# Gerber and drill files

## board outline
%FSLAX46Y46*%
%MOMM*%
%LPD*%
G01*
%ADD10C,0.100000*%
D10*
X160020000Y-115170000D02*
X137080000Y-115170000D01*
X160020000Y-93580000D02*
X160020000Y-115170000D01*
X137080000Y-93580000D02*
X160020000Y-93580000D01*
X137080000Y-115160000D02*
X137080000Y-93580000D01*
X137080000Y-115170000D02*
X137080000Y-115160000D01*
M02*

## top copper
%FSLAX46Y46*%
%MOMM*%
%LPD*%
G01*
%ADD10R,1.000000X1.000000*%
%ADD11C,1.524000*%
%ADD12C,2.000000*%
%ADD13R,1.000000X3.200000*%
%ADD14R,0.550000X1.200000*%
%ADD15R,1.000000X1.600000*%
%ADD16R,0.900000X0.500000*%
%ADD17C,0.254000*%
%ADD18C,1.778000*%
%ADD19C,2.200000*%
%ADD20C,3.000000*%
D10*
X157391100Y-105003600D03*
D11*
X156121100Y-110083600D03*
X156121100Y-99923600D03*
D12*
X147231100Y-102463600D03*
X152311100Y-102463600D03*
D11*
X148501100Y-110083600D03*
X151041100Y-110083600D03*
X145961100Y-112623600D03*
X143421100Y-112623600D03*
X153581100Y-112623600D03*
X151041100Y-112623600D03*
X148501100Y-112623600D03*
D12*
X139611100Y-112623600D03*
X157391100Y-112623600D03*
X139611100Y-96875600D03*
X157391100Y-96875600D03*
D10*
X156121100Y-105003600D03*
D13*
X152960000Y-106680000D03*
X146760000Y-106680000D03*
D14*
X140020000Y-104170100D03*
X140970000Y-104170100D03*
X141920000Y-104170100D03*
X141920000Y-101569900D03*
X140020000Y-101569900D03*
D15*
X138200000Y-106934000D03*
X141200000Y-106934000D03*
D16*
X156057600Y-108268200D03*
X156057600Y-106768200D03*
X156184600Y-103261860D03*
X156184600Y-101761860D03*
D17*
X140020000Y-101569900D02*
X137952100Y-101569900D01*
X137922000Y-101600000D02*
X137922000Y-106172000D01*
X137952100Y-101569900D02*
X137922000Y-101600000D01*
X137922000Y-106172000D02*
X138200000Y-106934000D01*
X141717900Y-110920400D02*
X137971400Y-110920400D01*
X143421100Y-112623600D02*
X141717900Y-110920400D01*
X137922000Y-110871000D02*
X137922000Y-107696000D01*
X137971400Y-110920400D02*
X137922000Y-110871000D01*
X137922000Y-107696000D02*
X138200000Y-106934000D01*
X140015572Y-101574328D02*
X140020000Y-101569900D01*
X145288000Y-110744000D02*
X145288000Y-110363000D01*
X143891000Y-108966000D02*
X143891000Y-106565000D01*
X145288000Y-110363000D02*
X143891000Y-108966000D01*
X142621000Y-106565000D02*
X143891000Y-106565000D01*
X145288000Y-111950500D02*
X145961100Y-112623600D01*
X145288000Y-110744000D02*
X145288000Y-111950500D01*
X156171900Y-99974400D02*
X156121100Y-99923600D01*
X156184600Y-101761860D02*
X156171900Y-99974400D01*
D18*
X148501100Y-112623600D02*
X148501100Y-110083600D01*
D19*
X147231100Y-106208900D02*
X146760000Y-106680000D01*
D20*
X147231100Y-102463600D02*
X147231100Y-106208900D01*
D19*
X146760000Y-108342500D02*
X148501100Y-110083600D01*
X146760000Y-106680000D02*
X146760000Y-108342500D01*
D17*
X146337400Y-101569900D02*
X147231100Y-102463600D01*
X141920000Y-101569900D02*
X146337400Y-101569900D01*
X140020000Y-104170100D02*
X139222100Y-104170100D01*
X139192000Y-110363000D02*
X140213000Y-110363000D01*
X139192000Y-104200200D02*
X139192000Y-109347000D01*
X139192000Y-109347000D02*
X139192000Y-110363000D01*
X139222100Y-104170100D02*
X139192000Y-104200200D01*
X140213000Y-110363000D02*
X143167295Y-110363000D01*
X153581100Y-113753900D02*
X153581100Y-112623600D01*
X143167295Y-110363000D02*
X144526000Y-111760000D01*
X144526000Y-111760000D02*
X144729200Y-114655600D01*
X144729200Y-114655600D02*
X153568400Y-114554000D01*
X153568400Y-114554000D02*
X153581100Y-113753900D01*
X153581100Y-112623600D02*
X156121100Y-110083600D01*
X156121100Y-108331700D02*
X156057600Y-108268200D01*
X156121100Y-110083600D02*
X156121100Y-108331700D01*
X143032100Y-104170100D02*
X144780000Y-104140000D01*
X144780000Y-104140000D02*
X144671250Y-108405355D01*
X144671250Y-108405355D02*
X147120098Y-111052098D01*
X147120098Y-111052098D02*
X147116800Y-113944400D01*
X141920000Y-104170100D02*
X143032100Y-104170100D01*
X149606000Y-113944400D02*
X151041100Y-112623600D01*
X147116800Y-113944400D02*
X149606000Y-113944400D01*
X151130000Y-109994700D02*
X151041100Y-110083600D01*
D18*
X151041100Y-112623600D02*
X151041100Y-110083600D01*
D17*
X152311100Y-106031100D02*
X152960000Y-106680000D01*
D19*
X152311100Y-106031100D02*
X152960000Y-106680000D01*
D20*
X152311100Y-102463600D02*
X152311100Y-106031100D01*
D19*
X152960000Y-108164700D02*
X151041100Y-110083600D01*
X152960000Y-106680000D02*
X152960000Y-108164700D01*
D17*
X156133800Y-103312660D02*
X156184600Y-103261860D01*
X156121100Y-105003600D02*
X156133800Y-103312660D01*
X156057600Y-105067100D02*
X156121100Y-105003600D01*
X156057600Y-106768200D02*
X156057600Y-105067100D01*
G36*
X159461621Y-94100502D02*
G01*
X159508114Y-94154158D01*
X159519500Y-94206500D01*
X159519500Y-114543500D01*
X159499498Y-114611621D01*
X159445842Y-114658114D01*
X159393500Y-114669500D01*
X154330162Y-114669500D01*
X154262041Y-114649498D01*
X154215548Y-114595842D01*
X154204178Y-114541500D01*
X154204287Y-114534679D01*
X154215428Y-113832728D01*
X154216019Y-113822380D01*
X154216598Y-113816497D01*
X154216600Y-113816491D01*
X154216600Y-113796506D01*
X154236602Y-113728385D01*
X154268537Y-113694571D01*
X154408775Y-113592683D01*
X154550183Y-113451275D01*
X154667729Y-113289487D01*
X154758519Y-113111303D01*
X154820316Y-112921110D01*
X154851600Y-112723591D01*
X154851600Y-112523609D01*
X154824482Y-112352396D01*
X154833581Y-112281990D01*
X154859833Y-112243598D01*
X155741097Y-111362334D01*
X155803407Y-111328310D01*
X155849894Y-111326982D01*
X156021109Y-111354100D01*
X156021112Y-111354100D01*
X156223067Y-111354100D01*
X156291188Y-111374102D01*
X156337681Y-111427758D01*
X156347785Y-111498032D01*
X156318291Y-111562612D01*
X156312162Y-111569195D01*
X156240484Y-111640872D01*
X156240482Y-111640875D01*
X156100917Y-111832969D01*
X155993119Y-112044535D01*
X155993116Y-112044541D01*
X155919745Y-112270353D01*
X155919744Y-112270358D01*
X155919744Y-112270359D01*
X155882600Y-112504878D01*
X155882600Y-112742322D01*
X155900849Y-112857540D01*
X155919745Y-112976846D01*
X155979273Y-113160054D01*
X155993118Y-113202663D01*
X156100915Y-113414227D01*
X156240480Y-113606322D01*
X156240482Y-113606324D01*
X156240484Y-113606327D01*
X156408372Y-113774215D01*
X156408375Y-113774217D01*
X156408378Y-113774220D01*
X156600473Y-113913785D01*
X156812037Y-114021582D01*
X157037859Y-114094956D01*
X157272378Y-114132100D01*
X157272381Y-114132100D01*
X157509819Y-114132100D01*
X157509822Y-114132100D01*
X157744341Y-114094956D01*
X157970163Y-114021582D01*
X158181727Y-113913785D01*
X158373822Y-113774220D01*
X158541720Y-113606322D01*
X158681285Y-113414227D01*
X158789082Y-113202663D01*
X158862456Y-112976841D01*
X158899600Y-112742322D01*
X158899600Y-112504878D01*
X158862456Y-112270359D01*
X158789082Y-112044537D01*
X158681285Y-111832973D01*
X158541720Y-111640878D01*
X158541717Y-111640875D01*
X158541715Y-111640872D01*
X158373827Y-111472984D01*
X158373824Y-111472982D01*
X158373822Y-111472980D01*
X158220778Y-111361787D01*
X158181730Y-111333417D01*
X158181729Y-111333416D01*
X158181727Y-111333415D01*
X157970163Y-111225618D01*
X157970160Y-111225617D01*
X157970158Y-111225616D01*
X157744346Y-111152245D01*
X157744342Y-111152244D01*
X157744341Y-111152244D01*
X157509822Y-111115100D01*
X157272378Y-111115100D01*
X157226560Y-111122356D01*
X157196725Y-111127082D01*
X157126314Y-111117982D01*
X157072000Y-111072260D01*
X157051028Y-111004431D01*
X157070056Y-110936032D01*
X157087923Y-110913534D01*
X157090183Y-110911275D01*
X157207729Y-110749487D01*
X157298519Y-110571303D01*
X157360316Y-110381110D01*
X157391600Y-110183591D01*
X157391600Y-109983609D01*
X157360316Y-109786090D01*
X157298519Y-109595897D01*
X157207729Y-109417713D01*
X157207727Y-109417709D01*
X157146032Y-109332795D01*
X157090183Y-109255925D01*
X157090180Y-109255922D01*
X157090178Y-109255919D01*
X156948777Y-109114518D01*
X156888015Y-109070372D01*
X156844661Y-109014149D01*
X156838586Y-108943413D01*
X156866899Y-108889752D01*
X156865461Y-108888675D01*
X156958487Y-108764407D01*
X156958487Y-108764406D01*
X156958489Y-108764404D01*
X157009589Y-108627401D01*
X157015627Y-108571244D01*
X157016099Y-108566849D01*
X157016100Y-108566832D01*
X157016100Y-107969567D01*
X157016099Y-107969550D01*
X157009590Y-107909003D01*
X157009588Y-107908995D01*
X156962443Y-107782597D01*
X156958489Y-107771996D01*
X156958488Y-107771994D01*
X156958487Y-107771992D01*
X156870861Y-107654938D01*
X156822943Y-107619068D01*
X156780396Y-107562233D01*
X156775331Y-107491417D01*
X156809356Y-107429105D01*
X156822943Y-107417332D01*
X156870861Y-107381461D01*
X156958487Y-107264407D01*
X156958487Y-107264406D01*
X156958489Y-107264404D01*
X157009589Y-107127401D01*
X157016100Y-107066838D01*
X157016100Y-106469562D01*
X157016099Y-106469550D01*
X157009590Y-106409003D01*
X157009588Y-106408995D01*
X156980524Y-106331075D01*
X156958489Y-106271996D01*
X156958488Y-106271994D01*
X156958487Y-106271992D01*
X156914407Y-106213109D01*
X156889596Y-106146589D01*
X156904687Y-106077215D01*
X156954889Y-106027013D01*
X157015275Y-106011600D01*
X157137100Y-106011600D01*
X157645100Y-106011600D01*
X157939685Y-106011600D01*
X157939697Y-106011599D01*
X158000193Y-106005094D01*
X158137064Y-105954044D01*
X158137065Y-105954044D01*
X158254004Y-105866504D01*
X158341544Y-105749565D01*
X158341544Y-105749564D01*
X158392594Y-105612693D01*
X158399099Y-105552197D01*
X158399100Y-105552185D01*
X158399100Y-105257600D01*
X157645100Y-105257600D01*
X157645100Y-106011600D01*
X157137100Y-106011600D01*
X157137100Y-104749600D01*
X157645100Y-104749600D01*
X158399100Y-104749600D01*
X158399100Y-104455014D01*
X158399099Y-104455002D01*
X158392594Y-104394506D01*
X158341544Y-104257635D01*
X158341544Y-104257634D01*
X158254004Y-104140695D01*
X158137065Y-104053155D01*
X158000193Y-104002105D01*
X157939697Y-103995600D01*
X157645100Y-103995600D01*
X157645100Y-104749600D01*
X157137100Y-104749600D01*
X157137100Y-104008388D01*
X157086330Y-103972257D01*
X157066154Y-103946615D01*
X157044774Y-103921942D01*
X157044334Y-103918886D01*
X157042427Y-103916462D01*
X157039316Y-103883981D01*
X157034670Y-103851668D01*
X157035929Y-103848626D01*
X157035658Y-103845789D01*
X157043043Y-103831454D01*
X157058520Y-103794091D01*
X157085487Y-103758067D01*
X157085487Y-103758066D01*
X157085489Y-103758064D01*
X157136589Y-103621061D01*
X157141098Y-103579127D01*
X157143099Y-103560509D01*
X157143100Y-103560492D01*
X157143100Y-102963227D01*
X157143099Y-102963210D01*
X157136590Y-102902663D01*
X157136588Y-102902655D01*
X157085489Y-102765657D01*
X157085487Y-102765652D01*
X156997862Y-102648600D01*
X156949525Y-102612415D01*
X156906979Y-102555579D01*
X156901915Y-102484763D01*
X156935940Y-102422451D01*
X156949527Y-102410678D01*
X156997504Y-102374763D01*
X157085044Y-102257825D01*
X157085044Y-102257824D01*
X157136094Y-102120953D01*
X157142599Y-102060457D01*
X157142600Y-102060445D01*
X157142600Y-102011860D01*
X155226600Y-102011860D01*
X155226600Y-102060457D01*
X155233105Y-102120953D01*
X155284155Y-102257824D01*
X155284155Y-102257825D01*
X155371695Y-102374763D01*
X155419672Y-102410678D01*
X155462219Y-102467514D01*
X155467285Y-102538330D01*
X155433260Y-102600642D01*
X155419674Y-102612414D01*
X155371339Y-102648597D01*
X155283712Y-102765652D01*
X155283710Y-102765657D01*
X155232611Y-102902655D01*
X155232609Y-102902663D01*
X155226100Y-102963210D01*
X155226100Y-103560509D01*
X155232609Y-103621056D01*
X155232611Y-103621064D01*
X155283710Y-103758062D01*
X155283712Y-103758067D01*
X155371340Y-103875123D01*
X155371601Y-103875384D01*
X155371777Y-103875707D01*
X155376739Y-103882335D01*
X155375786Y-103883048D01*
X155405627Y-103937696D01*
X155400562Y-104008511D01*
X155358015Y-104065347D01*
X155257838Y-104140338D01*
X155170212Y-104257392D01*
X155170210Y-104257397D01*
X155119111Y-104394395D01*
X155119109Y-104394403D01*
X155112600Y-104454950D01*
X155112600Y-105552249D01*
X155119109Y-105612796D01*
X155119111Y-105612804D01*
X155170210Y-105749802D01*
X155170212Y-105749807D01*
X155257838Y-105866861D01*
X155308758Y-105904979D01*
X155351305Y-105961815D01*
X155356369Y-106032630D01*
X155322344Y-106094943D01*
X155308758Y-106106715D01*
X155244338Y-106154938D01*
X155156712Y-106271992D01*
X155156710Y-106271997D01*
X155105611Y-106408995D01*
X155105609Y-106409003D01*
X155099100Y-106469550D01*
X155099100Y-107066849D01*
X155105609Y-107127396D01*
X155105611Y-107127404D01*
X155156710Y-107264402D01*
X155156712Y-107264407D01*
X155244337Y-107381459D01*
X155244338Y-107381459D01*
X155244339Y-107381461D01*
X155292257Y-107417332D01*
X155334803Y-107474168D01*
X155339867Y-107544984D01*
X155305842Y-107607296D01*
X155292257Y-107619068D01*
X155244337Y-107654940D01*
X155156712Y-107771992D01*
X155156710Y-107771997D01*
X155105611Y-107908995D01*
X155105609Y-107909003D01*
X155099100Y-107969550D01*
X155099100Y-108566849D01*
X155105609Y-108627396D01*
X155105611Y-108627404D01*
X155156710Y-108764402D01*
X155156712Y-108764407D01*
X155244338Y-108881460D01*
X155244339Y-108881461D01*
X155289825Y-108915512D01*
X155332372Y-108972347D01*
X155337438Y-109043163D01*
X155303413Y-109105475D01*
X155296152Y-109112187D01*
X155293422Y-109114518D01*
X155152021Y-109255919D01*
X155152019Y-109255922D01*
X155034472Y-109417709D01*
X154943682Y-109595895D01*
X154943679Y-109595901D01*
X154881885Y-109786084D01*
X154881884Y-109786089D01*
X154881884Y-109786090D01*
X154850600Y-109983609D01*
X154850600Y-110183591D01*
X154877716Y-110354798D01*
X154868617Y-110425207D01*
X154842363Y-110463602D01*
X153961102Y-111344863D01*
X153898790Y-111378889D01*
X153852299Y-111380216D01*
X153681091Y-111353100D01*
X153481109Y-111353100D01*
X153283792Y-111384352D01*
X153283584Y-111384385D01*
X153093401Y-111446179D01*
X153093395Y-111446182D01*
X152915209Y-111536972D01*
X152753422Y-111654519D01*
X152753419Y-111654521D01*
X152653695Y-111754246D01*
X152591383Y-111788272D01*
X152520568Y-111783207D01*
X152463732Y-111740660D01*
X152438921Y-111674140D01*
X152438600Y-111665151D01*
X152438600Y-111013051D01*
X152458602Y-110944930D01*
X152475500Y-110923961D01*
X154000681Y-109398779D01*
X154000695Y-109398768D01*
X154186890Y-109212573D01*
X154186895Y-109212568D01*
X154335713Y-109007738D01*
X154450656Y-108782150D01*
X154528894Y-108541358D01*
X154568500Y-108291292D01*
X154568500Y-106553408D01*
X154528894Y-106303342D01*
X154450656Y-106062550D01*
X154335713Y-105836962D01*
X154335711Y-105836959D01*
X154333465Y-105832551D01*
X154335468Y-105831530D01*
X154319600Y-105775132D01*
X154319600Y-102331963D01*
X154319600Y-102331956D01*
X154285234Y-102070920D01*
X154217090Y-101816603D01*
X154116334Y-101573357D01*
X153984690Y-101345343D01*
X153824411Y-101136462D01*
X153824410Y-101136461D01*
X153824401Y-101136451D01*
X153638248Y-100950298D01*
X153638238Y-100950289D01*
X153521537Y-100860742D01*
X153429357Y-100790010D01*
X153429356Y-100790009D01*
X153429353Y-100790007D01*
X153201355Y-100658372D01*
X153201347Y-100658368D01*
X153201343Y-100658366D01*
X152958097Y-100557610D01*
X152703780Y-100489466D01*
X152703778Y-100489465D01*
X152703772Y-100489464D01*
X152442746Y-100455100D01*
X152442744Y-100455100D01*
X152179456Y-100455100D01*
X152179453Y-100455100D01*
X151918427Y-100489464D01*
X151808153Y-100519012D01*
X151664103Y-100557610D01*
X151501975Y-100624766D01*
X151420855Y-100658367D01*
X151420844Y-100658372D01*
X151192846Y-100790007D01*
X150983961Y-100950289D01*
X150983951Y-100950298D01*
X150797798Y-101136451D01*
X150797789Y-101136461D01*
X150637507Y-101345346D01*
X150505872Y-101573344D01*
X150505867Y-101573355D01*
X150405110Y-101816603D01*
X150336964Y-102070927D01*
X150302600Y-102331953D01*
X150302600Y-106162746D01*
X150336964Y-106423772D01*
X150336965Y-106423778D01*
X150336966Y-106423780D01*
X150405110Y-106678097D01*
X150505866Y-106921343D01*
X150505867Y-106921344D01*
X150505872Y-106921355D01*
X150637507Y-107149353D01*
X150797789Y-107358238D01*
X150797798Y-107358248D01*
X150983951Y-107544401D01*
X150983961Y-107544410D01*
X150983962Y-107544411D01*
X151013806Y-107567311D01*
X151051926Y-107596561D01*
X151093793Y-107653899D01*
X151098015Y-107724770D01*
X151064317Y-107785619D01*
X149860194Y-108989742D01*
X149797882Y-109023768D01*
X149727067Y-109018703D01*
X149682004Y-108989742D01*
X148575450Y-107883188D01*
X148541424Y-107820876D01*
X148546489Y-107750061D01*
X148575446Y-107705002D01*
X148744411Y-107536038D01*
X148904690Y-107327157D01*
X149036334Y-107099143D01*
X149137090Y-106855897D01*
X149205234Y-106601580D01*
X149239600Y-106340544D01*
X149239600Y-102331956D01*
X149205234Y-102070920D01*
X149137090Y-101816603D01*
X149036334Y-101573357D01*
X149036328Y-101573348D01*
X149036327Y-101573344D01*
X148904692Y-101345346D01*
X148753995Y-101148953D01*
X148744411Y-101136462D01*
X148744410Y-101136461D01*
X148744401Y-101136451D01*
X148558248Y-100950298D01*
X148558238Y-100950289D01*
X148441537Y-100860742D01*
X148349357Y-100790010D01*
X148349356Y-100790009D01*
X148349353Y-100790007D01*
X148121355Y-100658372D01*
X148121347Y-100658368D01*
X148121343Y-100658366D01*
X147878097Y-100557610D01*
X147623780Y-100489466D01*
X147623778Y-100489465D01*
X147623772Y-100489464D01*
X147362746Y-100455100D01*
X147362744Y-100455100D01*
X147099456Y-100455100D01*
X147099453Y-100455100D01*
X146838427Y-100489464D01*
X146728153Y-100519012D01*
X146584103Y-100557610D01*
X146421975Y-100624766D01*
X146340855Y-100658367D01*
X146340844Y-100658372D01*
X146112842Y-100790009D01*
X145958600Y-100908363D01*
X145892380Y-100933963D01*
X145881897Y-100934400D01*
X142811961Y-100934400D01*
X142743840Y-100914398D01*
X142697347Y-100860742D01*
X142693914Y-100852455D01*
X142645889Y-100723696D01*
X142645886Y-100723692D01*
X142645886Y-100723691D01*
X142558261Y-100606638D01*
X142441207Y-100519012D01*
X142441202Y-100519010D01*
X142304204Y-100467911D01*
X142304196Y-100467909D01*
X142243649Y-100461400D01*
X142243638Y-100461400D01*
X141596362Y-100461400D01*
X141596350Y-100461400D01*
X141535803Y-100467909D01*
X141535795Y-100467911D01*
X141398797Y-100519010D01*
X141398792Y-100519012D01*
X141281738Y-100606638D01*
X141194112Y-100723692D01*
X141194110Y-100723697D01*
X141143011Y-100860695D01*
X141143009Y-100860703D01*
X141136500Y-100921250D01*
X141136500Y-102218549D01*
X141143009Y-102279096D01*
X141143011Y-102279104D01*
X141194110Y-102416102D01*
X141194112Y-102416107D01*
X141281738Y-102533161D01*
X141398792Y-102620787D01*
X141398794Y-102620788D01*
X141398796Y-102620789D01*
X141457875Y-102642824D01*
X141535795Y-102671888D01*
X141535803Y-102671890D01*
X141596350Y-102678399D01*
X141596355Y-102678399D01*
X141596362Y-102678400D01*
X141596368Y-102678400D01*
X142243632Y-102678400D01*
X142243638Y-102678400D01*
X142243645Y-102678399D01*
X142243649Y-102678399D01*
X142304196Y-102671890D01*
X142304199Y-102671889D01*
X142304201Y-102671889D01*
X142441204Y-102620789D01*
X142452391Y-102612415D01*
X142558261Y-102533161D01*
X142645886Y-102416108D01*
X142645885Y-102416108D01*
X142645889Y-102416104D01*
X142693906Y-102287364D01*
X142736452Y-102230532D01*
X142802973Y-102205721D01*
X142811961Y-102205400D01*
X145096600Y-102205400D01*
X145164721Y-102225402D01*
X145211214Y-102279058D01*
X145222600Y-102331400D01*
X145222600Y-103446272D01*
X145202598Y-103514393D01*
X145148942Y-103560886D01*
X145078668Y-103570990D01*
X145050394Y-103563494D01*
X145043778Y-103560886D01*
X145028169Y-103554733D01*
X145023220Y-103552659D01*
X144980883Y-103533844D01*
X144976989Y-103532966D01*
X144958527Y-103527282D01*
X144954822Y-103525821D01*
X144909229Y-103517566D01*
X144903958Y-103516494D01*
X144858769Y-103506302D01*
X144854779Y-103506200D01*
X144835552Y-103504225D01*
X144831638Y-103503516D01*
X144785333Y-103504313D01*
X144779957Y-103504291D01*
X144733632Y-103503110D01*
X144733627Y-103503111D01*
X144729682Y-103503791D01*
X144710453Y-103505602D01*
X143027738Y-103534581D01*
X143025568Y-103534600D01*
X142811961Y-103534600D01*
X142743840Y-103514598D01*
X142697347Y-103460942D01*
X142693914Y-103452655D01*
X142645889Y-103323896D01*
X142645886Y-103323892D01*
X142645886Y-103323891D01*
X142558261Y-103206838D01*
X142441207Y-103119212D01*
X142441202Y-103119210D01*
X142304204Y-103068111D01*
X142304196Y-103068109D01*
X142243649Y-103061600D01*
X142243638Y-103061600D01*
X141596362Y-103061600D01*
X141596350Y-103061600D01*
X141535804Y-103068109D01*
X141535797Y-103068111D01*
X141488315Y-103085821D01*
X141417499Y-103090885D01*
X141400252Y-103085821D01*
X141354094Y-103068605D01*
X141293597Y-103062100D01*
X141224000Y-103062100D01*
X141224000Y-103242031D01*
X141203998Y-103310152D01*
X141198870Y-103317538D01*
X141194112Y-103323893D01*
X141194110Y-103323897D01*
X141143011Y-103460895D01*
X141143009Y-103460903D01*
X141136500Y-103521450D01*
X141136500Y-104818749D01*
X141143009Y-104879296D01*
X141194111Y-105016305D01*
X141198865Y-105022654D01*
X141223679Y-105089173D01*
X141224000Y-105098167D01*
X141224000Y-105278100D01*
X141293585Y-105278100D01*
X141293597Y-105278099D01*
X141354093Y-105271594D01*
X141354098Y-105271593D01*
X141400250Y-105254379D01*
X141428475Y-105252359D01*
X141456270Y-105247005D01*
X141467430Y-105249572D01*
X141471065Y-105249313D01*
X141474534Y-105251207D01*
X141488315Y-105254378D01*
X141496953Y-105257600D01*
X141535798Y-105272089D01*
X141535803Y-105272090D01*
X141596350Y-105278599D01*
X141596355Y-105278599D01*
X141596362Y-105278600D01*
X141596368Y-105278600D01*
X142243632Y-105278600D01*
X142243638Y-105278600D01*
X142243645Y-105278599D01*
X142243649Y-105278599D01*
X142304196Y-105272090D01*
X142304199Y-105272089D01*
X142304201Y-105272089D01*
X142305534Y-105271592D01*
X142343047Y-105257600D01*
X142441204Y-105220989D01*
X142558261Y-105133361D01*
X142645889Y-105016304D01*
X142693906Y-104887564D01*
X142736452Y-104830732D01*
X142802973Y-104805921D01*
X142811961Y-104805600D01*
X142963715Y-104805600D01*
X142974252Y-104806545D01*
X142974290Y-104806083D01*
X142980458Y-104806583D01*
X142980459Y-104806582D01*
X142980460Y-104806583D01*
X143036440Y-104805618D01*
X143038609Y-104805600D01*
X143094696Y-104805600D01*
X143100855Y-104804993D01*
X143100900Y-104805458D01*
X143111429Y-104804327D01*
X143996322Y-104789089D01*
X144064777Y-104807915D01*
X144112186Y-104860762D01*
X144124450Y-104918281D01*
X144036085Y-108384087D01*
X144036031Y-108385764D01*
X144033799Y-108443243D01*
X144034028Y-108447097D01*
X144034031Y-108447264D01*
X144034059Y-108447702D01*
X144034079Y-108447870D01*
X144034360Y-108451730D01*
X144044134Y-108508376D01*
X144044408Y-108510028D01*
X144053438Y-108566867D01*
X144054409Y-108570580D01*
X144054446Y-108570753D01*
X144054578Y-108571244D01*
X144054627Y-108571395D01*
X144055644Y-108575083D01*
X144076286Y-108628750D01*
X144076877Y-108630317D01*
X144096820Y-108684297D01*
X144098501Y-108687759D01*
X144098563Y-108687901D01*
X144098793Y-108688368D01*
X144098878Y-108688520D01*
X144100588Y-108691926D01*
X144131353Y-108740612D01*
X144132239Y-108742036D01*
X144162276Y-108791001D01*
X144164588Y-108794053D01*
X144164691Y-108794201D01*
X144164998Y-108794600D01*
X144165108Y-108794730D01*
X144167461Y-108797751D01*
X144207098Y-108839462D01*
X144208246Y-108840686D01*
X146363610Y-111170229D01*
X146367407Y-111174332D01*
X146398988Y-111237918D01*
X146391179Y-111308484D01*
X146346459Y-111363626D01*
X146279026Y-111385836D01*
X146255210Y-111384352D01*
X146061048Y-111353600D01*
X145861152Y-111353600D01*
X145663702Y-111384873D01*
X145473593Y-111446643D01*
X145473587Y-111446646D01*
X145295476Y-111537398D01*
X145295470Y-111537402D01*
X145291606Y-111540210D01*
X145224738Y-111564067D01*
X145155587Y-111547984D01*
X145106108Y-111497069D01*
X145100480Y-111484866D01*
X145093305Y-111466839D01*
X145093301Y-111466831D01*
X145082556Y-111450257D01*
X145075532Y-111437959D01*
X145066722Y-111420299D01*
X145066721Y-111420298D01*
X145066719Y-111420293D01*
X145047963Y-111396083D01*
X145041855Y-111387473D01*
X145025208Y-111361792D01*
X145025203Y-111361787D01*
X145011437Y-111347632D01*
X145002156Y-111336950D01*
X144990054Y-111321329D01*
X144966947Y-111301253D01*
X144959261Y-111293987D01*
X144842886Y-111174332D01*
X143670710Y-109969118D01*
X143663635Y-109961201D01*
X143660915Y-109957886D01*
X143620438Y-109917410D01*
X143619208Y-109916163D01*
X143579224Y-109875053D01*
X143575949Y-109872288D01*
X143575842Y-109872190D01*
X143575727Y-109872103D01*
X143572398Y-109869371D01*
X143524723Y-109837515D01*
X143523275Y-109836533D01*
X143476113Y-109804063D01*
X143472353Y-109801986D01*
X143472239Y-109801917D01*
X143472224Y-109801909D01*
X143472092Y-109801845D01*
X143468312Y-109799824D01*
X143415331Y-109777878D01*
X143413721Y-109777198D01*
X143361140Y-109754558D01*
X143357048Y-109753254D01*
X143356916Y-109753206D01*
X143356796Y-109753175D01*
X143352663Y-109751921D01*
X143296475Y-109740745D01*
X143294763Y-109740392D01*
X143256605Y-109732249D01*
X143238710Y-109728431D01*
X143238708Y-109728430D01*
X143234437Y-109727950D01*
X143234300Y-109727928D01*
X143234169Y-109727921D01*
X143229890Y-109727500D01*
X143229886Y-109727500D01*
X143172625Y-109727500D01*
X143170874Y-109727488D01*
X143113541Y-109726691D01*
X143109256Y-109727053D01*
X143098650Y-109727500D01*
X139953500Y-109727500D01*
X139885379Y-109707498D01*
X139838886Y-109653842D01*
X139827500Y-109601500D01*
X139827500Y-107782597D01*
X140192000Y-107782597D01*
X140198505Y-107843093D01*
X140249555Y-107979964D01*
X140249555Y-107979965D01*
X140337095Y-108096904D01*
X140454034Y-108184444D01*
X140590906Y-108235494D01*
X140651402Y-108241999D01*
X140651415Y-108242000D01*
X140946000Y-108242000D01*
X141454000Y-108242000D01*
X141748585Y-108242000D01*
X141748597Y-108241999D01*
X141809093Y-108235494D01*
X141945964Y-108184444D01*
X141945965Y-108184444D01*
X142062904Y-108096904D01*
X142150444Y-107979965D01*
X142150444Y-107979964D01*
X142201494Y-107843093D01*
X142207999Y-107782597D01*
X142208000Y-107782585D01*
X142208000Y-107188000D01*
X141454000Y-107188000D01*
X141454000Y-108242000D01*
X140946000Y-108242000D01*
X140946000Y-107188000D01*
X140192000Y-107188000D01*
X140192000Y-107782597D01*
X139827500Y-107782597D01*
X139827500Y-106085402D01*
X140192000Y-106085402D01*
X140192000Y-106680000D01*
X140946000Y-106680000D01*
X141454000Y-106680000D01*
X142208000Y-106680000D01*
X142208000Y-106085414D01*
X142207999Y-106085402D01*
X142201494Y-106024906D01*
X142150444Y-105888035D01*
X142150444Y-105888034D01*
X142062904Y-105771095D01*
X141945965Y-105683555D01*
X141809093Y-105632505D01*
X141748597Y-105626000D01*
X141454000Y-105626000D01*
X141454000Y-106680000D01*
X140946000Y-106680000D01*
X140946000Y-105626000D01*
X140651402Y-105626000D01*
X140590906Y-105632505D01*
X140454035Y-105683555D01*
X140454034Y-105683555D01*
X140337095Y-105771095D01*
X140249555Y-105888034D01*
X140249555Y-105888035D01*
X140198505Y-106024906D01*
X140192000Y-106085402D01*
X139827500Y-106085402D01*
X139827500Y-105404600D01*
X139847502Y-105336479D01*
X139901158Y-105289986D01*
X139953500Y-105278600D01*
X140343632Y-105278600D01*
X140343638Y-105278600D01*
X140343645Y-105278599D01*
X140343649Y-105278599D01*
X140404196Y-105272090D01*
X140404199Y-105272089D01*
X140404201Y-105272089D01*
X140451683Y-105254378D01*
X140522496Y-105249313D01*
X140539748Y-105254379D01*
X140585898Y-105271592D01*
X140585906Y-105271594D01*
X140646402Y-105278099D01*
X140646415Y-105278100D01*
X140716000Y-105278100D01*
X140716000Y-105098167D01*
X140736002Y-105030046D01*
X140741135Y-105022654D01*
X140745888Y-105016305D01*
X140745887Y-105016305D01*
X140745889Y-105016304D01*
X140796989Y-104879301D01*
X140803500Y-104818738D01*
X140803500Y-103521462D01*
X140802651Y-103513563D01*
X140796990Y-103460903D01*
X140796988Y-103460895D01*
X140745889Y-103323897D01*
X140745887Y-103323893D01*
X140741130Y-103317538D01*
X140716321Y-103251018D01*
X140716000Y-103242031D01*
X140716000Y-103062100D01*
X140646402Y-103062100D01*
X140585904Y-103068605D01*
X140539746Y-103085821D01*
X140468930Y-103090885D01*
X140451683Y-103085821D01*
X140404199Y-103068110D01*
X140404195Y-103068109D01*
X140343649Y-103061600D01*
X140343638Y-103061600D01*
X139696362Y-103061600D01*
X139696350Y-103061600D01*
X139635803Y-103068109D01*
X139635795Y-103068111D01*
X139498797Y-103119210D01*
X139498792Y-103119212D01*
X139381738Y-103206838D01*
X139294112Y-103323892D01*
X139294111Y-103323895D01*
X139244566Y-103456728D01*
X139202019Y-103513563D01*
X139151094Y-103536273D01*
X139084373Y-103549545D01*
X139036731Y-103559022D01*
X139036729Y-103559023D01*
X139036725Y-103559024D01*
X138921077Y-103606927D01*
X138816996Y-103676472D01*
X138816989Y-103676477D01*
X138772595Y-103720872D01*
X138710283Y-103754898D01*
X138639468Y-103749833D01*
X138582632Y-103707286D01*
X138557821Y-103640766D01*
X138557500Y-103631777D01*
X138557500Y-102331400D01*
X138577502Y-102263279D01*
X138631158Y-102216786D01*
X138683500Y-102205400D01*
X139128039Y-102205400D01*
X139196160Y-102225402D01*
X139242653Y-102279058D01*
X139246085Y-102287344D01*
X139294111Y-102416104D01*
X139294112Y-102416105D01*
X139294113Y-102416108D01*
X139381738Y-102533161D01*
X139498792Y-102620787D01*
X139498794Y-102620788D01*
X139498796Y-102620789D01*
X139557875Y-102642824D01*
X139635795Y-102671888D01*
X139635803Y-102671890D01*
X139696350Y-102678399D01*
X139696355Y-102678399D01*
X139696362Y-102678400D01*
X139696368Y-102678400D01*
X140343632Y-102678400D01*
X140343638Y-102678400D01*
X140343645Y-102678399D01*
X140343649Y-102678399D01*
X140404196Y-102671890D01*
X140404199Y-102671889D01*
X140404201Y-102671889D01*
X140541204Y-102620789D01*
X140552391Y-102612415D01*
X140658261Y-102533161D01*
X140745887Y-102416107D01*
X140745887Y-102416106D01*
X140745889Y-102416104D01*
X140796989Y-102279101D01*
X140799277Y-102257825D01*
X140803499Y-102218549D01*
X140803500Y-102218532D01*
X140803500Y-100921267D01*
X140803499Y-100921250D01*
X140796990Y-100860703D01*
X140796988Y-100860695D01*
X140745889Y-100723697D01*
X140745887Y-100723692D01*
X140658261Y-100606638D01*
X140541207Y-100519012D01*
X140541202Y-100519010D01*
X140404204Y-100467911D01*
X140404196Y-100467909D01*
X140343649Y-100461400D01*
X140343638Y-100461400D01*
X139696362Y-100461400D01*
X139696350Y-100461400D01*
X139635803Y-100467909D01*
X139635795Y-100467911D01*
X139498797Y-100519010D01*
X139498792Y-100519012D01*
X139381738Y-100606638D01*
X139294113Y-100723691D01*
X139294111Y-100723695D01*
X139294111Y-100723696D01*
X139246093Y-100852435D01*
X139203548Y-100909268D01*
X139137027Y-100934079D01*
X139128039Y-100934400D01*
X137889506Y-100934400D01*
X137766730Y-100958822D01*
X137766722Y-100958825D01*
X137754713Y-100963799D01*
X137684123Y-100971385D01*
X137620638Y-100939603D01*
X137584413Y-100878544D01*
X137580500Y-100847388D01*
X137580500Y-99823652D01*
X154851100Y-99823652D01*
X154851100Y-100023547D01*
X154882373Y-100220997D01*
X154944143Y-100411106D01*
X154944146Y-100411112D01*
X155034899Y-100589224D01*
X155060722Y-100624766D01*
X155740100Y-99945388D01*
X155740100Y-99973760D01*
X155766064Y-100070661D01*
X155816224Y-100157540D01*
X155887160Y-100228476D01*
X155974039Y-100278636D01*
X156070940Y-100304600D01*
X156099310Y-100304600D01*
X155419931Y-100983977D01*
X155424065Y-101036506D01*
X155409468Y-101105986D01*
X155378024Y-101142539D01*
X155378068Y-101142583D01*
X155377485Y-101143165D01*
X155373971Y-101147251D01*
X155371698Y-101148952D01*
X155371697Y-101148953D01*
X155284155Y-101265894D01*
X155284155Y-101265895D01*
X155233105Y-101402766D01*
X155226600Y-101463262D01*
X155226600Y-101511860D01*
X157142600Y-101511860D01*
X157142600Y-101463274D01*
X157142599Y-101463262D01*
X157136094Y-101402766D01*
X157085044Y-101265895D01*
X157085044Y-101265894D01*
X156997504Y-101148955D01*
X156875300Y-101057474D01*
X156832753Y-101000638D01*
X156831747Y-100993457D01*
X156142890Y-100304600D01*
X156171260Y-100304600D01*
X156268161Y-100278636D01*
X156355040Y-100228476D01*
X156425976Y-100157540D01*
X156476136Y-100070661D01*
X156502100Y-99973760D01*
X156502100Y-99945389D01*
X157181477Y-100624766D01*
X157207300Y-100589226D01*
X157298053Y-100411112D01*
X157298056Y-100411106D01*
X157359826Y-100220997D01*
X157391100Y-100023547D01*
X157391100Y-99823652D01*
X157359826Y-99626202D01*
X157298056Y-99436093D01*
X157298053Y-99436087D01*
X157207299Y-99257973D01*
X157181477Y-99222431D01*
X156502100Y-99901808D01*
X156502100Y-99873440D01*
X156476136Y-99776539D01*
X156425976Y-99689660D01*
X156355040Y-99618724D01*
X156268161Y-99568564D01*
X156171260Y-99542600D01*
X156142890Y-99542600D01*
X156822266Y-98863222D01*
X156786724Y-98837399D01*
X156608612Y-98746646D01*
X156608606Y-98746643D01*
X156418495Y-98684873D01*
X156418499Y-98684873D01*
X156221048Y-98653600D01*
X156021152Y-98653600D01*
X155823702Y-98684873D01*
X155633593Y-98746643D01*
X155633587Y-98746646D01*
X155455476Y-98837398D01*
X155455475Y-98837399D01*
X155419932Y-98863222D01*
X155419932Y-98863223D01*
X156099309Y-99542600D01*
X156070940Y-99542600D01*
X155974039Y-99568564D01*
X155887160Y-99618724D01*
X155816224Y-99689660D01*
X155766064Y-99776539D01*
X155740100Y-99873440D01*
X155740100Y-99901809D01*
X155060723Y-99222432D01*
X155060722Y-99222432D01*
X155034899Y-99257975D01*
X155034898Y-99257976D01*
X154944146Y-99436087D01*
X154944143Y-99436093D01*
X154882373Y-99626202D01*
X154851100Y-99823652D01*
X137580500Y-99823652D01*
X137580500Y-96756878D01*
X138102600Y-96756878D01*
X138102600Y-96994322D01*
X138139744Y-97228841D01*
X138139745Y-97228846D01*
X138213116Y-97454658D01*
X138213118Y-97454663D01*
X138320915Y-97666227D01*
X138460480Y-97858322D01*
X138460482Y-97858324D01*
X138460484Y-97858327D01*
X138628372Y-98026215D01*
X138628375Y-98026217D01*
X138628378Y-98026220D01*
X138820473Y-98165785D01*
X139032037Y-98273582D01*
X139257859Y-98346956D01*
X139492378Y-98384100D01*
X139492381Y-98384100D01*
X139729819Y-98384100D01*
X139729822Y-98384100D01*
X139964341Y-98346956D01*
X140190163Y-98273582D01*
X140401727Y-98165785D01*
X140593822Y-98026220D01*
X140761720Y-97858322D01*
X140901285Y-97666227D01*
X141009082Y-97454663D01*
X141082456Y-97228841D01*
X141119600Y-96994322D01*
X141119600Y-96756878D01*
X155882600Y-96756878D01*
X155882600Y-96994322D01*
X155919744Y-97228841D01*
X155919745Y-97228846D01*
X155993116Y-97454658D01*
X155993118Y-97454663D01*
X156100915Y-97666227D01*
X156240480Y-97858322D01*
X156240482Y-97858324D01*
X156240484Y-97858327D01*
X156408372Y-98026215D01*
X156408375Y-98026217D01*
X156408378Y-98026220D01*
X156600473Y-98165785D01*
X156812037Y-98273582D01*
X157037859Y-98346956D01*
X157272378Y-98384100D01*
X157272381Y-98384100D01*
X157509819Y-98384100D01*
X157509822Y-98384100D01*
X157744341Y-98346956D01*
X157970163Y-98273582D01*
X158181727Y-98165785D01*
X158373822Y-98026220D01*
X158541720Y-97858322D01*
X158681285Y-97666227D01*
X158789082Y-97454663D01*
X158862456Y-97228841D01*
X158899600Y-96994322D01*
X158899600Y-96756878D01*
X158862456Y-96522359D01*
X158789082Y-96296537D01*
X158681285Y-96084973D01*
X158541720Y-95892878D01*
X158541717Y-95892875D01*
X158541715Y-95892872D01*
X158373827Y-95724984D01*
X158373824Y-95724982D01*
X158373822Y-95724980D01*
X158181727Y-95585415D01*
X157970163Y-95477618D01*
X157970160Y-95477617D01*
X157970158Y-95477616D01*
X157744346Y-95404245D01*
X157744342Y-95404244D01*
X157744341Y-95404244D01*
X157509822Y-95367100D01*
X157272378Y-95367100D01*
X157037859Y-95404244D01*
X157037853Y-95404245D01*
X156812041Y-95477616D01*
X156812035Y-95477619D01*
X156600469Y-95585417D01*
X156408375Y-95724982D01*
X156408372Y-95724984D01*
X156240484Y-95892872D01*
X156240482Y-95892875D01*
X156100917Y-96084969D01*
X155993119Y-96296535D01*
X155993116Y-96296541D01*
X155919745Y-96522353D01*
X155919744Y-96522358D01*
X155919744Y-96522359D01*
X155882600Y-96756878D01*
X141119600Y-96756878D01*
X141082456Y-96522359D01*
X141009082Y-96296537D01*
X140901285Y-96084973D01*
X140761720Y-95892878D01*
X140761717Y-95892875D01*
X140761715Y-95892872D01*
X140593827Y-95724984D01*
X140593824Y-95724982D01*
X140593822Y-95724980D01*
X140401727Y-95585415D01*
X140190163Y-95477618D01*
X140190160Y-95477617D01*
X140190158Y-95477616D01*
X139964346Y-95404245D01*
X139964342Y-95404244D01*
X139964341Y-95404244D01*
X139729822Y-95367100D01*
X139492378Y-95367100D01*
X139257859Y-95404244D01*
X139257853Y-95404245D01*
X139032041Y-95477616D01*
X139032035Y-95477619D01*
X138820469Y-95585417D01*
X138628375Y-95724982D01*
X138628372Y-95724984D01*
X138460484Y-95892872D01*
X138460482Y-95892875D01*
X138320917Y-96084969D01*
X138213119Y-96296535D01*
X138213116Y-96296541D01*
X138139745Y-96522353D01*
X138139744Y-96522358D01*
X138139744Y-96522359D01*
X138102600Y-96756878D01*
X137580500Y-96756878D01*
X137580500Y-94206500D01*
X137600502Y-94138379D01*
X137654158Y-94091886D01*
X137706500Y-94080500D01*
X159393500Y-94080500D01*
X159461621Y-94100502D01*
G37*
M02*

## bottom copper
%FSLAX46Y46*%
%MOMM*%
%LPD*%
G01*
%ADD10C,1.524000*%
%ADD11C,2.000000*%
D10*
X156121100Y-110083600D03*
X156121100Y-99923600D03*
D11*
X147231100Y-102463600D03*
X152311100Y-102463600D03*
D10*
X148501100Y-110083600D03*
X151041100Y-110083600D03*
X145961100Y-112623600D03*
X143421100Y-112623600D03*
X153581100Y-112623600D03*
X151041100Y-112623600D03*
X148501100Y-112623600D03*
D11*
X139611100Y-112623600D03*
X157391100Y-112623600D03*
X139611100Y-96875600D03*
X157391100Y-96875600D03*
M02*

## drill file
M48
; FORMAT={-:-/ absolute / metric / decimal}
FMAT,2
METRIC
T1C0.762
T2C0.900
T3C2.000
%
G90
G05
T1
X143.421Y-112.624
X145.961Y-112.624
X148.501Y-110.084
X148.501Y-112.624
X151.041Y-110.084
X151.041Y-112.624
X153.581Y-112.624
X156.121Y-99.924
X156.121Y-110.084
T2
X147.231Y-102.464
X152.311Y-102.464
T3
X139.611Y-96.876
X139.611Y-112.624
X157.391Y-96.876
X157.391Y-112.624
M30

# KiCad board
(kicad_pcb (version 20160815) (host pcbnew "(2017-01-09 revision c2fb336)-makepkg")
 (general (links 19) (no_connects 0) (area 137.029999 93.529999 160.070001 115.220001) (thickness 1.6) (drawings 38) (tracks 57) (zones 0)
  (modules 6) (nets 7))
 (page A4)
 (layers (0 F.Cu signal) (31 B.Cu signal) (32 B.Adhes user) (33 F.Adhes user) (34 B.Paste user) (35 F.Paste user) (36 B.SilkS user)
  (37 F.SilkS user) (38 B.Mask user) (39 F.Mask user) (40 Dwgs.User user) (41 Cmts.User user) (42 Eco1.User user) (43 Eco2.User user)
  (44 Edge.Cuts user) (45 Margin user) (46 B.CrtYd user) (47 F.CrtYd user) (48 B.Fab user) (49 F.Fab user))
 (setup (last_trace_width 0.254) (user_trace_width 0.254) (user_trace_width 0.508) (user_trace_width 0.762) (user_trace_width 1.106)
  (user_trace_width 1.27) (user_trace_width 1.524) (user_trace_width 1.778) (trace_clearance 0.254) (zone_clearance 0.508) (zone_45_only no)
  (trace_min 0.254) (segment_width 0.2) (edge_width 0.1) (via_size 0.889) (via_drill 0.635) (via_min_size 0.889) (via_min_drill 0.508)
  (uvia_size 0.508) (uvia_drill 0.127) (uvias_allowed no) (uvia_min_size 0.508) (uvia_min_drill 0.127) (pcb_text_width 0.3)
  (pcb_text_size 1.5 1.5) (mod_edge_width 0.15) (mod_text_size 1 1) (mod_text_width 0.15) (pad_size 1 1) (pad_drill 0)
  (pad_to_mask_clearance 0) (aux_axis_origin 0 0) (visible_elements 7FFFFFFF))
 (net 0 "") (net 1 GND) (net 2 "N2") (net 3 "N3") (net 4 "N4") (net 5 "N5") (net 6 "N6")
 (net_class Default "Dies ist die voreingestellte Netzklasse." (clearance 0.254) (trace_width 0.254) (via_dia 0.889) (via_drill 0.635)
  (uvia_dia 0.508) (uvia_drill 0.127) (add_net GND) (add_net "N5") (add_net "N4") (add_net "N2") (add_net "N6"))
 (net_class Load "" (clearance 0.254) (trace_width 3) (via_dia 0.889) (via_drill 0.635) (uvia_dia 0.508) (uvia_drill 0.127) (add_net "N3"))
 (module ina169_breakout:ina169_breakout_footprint (layer F.Cu) (at 148.5011 105.0036)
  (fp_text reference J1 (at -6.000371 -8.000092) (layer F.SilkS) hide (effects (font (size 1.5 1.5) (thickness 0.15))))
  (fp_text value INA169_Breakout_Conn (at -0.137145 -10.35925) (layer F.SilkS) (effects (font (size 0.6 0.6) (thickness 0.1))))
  (pad 2 smd rect (at 8.89 0) (size 1 1) (layers F.Cu F.Paste F.Mask) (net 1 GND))
  (pad 5 thru_hole circle (at 7.62 5.08) (size 1.524 1.524) (drill 0.762) (layers *.Cu *.Mask F.SilkS) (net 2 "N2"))
  (pad 2 thru_hole circle (at 7.62 -5.08) (size 1.524 1.524) (drill 0.762) (layers *.Cu *.Mask F.SilkS) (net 1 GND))
  (pad 3 thru_hole circle (at -1.27 -2.54) (size 2 2) (drill 0.9) (layers *.Cu *.Mask F.SilkS) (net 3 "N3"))
  (pad 4 thru_hole circle (at 3.81 -2.54) (size 2 2) (drill 0.9) (layers *.Cu *.Mask F.SilkS) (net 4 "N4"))
  (pad 3 thru_hole circle (at 0 5.08) (size 1.524 1.524) (drill 0.762) (layers *.Cu *.Mask F.SilkS) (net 3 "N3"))
  (pad 4 thru_hole circle (at 2.54 5.08) (size 1.524 1.524) (drill 0.762) (layers *.Cu *.Mask F.SilkS) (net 4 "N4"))
  (pad 2 thru_hole circle (at -2.54 7.62) (size 1.524 1.524) (drill 0.762) (layers *.Cu *.Mask F.SilkS) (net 1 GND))
  (pad 1 thru_hole circle (at -5.08 7.62) (size 1.524 1.524) (drill 0.762) (layers *.Cu *.Mask F.SilkS) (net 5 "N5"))
  (pad 5 thru_hole circle (at 5.08 7.62) (size 1.524 1.524) (drill 0.762) (layers *.Cu *.Mask F.SilkS) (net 2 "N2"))
  (pad 4 thru_hole circle (at 2.54 7.62) (size 1.524 1.524) (drill 0.762) (layers *.Cu *.Mask F.SilkS) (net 4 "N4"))
  (pad 3 thru_hole circle (at 0 7.62) (size 1.524 1.524) (drill 0.762) (layers *.Cu *.Mask F.SilkS) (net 3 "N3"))
  (pad "" thru_hole circle (at -8.89 7.62) (size 2 2) (drill 2) (layers *.Cu *.Mask F.SilkS))
  (pad "" thru_hole circle (at 8.89 7.62) (size 2 2) (drill 2) (layers *.Cu *.Mask F.SilkS))
  (pad "" thru_hole circle (at -8.89 -8.128) (size 2 2) (drill 2) (layers *.Cu *.Mask F.SilkS))
  (pad "" thru_hole circle (at 8.89 -8.128) (size 2 2) (drill 2) (layers *.Cu *.Mask F.SilkS))
  (pad 6 smd rect (at 7.62 0) (size 1 1) (layers F.Cu F.Paste F.Mask)))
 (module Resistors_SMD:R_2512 (layer F.Cu) (at 149.86 106.68 180)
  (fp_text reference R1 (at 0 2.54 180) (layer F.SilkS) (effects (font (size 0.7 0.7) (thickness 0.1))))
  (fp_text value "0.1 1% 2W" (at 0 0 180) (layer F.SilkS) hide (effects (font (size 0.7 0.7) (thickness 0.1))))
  (pad 1 smd rect (at -3.1 0 180) (size 1 3.2) (layers F.Cu F.Paste F.Mask) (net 4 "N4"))
  (pad 2 smd rect (at 3.1 0 180) (size 1 3.2) (layers F.Cu F.Paste F.Mask) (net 3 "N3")))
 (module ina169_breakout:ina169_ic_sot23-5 (layer F.Cu) (at 140.97 102.87)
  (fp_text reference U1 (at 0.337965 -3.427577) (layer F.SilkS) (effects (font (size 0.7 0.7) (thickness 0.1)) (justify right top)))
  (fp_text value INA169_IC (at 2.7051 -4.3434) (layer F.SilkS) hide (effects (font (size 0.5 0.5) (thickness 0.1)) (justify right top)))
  (pad 1 smd rect (at -0.95 1.3001) (size 0.55 1.2) (layers F.Cu F.Paste F.Mask) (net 2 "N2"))
  (pad 2 smd rect (at 0 1.3001) (size 0.55 1.2) (layers F.Cu F.Paste F.Mask) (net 1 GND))
  (pad 3 smd rect (at 0.95 1.3001) (size 0.55 1.2) (layers F.Cu F.Paste F.Mask) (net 4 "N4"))
  (pad 4 smd rect (at 0.95 -1.3001) (size 0.55 1.2) (layers F.Cu F.Paste F.Mask) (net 3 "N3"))
  (pad 5 smd rect (at -0.95 -1.3001) (size 0.55 1.2) (layers F.Cu F.Paste F.Mask) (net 5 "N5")))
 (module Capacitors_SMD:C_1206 (layer F.Cu) (at 139.7 106.934)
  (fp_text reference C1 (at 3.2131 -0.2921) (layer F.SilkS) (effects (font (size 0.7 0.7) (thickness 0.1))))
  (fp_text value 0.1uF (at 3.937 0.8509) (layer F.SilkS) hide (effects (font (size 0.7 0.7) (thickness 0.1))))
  (pad 1 smd rect (at -1.5 0) (size 1 1.6) (layers F.Cu F.Paste F.Mask) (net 5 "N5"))
  (pad 2 smd rect (at 1.5 0) (size 1 1.6) (layers F.Cu F.Paste F.Mask) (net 1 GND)))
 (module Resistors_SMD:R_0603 (layer F.Cu) (at 156.0576 107.5182 90)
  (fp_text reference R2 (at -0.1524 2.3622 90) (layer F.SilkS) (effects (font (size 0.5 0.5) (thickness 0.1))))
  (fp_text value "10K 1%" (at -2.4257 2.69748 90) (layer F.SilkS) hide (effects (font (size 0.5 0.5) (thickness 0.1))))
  (pad 1 smd rect (at -0.75 0 90) (size 0.5 0.9) (layers F.Cu F.Paste F.Mask) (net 2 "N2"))
  (pad 2 smd rect (at 0.75 0 90) (size 0.5 0.9) (layers F.Cu F.Paste F.Mask) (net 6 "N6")))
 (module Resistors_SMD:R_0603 (layer F.Cu) (at 156.1846 102.51186 90)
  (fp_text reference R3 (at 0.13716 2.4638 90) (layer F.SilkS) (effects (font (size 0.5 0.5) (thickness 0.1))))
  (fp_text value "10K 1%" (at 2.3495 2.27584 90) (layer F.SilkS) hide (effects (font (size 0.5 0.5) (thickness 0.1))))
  (pad 1 smd rect (at -0.75 0 90) (size 0.5 0.9) (layers F.Cu F.Paste F.Mask) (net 6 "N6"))
  (pad 2 smd rect (at 0.75 0 90) (size 0.5 0.9) (layers F.Cu F.Paste F.Mask) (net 1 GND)))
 (gr_line (start 160.02 115.17) (end 137.08 115.17) (angle 90) (layer Edge.Cuts) (width 0.1))
 (gr_line (start 160.02 93.58) (end 160.02 115.17) (angle 90) (layer Edge.Cuts) (width 0.1))
 (gr_line (start 137.08 93.58) (end 160.02 93.58) (angle 90) (layer Edge.Cuts) (width 0.1))
 (gr_line (start 137.08 115.16) (end 137.08 93.58) (angle 90) (layer Edge.Cuts) (width 0.1))
 (gr_line (start 137.08 115.17) (end 137.08 115.16) (angle 90) (layer Edge.Cuts) (width 0.1))
 (segment (start 140.02 101.5699) (end 137.9521 101.5699) (width 0.254) (layer F.Cu) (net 5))
 (segment (start 137.922 101.6) (end 137.922 106.172) (width 0.254) (layer F.Cu) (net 5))
 (segment (start 137.9521 101.5699) (end 137.922 101.6) (width 0.254) (layer F.Cu) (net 5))
 (segment (start 137.922 106.172) (end 138.2 106.934) (width 0.254) (layer F.Cu) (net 5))
 (segment (start 141.7179 110.9204) (end 137.9714 110.9204) (width 0.254) (layer F.Cu) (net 5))
 (segment (start 143.4211 112.6236) (end 141.7179 110.9204) (width 0.254) (layer F.Cu) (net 5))
 (segment (start 137.922 110.871) (end 137.922 107.696) (width 0.254) (layer F.Cu) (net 5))
 (segment (start 137.9714 110.9204) (end 137.922 110.871) (width 0.254) (layer F.Cu) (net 5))
 (segment (start 137.922 107.696) (end 138.2 106.934) (width 0.254) (layer F.Cu) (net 5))
 (segment (start 140.015572 101.574328) (end 140.02 101.5699) (width 0.254) (layer F.Cu) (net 5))
 (segment (start 145.288 110.744) (end 145.288 110.363) (width 0.254) (layer F.Cu) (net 1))
 (segment (start 143.891 108.966) (end 143.891 106.565) (width 0.254) (layer F.Cu) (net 1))
 (segment (start 145.288 110.363) (end 143.891 108.966) (width 0.254) (layer F.Cu) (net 1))
 (segment (start 142.621 106.565) (end 143.891 106.565) (width 0.254) (layer F.Cu) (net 1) (status 10))
 (segment (start 145.288 111.9505) (end 145.9611 112.6236) (width 0.254) (layer F.Cu) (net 1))
 (segment (start 145.288 110.744) (end 145.288 111.9505) (width 0.254) (layer F.Cu) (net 1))
 (segment (start 156.1719 99.9744) (end 156.1211 99.9236) (width 0.254) (layer F.Cu) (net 1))
 (segment (start 156.1846 101.76186) (end 156.1719 99.9744) (width 0.254) (layer F.Cu) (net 1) (status 10))
 (segment (start 148.5011 112.6236) (end 148.5011 110.0836) (width 1.778) (layer F.Cu) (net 3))
 (segment (start 147.2311 106.2089) (end 146.76 106.68) (width 2.2) (layer F.Cu) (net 3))
 (segment (start 147.2311 102.4636) (end 147.2311 106.2089) (width 3) (layer F.Cu) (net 3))
 (segment (start 146.76 108.3425) (end 148.5011 110.0836) (width 2.2) (layer F.Cu) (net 3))
 (segment (start 146.76 106.68) (end 146.76 108.3425) (width 2.2) (layer F.Cu) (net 3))
 (segment (start 146.3374 101.5699) (end 147.2311 102.4636) (width 0.254) (layer F.Cu) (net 3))
 (segment (start 141.92 101.5699) (end 146.3374 101.5699) (width 0.254) (layer F.Cu) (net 3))
 (segment (start 140.02 104.1701) (end 139.2221 104.1701) (width 0.254) (layer F.Cu) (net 2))
 (segment (start 139.192 110.363) (end 140.213 110.363) (width 0.254) (layer F.Cu) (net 2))
 (segment (start 139.192 104.2002) (end 139.192 109.347) (width 0.254) (layer F.Cu) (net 2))
 (segment (start 139.192 109.347) (end 139.192 110.363) (width 0.254) (layer F.Cu) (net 2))
 (segment (start 139.2221 104.1701) (end 139.192 104.2002) (width 0.254) (layer F.Cu) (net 2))
 (segment (start 140.213 110.363) (end 143.167295 110.363) (width 0.254) (layer F.Cu) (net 2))
 (segment (start 153.5811 113.7539) (end 153.5811 112.6236) (width 0.254) (layer F.Cu) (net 2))
 (segment (start 143.167295 110.363) (end 144.526 111.76) (width 0.254) (layer F.Cu) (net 2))
 (segment (start 144.526 111.76) (end 144.7292 114.6556) (width 0.254) (layer F.Cu) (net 2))
 (segment (start 144.7292 114.6556) (end 153.5684 114.554) (width 0.254) (layer F.Cu) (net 2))
 (segment (start 153.5684 114.554) (end 153.5811 113.7539) (width 0.254) (layer F.Cu) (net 2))
 (segment (start 153.5811 112.6236) (end 156.1211 110.0836) (width 0.254) (layer F.Cu) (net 2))
 (segment (start 156.1211 108.3317) (end 156.0576 108.2682) (width 0.254) (layer F.Cu) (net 2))
 (segment (start 156.1211 110.0836) (end 156.1211 108.3317) (width 0.254) (layer F.Cu) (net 2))
 (segment (start 143.0321 104.1701) (end 144.78 104.14) (width 0.254) (layer F.Cu) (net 4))
 (segment (start 144.78 104.14) (end 144.67125 108.405355) (width 0.254) (layer F.Cu) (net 4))
 (segment (start 144.67125 108.405355) (end 147.120098 111.052098) (width 0.254) (layer F.Cu) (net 4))
 (segment (start 147.120098 111.052098) (end 147.1168 113.9444) (width 0.254) (layer F.Cu) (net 4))
 (segment (start 141.92 104.1701) (end 143.0321 104.1701) (width 0.254) (layer F.Cu) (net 4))
 (segment (start 149.606 113.9444) (end 151.0411 112.6236) (width 0.254) (layer F.Cu) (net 4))
 (segment (start 147.1168 113.9444) (end 149.606 113.9444) (width 0.254) (layer F.Cu) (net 4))
 (segment (start 151.13 109.9947) (end 151.0411 110.0836) (width 0.254) (layer F.Cu) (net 4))
 (segment (start 151.0411 112.6236) (end 151.0411 110.0836) (width 1.778) (layer F.Cu) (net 4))
 (segment (start 152.3111 106.0311) (end 152.96 106.68) (width 0.254) (layer F.Cu) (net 4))
 (segment (start 152.3111 106.0311) (end 152.96 106.68) (width 2.2) (layer F.Cu) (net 4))
 (segment (start 152.3111 102.4636) (end 152.3111 106.0311) (width 3) (layer F.Cu) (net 4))
 (segment (start 152.96 108.1647) (end 151.0411 110.0836) (width 2.2) (layer F.Cu) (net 4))
 (segment (start 152.96 106.68) (end 152.96 108.1647) (width 2.2) (layer F.Cu) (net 4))
 (segment (start 156.1338 103.31266) (end 156.1846 103.26186) (width 0.254) (layer F.Cu) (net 6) (status 30))
 (segment (start 156.1211 105.0036) (end 156.1338 103.31266) (width 0.254) (layer F.Cu) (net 6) (status 20))
 (segment (start 156.0576 105.0671) (end 156.1211 105.0036) (width 0.254) (layer F.Cu) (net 6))
 (segment (start 156.0576 106.7682) (end 156.0576 105.0671) (width 0.254) (layer F.Cu) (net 6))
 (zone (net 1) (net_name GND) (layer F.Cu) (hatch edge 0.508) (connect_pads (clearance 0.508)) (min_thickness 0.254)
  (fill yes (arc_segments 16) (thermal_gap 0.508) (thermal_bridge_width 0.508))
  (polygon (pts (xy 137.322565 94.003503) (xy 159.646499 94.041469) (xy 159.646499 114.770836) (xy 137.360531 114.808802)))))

